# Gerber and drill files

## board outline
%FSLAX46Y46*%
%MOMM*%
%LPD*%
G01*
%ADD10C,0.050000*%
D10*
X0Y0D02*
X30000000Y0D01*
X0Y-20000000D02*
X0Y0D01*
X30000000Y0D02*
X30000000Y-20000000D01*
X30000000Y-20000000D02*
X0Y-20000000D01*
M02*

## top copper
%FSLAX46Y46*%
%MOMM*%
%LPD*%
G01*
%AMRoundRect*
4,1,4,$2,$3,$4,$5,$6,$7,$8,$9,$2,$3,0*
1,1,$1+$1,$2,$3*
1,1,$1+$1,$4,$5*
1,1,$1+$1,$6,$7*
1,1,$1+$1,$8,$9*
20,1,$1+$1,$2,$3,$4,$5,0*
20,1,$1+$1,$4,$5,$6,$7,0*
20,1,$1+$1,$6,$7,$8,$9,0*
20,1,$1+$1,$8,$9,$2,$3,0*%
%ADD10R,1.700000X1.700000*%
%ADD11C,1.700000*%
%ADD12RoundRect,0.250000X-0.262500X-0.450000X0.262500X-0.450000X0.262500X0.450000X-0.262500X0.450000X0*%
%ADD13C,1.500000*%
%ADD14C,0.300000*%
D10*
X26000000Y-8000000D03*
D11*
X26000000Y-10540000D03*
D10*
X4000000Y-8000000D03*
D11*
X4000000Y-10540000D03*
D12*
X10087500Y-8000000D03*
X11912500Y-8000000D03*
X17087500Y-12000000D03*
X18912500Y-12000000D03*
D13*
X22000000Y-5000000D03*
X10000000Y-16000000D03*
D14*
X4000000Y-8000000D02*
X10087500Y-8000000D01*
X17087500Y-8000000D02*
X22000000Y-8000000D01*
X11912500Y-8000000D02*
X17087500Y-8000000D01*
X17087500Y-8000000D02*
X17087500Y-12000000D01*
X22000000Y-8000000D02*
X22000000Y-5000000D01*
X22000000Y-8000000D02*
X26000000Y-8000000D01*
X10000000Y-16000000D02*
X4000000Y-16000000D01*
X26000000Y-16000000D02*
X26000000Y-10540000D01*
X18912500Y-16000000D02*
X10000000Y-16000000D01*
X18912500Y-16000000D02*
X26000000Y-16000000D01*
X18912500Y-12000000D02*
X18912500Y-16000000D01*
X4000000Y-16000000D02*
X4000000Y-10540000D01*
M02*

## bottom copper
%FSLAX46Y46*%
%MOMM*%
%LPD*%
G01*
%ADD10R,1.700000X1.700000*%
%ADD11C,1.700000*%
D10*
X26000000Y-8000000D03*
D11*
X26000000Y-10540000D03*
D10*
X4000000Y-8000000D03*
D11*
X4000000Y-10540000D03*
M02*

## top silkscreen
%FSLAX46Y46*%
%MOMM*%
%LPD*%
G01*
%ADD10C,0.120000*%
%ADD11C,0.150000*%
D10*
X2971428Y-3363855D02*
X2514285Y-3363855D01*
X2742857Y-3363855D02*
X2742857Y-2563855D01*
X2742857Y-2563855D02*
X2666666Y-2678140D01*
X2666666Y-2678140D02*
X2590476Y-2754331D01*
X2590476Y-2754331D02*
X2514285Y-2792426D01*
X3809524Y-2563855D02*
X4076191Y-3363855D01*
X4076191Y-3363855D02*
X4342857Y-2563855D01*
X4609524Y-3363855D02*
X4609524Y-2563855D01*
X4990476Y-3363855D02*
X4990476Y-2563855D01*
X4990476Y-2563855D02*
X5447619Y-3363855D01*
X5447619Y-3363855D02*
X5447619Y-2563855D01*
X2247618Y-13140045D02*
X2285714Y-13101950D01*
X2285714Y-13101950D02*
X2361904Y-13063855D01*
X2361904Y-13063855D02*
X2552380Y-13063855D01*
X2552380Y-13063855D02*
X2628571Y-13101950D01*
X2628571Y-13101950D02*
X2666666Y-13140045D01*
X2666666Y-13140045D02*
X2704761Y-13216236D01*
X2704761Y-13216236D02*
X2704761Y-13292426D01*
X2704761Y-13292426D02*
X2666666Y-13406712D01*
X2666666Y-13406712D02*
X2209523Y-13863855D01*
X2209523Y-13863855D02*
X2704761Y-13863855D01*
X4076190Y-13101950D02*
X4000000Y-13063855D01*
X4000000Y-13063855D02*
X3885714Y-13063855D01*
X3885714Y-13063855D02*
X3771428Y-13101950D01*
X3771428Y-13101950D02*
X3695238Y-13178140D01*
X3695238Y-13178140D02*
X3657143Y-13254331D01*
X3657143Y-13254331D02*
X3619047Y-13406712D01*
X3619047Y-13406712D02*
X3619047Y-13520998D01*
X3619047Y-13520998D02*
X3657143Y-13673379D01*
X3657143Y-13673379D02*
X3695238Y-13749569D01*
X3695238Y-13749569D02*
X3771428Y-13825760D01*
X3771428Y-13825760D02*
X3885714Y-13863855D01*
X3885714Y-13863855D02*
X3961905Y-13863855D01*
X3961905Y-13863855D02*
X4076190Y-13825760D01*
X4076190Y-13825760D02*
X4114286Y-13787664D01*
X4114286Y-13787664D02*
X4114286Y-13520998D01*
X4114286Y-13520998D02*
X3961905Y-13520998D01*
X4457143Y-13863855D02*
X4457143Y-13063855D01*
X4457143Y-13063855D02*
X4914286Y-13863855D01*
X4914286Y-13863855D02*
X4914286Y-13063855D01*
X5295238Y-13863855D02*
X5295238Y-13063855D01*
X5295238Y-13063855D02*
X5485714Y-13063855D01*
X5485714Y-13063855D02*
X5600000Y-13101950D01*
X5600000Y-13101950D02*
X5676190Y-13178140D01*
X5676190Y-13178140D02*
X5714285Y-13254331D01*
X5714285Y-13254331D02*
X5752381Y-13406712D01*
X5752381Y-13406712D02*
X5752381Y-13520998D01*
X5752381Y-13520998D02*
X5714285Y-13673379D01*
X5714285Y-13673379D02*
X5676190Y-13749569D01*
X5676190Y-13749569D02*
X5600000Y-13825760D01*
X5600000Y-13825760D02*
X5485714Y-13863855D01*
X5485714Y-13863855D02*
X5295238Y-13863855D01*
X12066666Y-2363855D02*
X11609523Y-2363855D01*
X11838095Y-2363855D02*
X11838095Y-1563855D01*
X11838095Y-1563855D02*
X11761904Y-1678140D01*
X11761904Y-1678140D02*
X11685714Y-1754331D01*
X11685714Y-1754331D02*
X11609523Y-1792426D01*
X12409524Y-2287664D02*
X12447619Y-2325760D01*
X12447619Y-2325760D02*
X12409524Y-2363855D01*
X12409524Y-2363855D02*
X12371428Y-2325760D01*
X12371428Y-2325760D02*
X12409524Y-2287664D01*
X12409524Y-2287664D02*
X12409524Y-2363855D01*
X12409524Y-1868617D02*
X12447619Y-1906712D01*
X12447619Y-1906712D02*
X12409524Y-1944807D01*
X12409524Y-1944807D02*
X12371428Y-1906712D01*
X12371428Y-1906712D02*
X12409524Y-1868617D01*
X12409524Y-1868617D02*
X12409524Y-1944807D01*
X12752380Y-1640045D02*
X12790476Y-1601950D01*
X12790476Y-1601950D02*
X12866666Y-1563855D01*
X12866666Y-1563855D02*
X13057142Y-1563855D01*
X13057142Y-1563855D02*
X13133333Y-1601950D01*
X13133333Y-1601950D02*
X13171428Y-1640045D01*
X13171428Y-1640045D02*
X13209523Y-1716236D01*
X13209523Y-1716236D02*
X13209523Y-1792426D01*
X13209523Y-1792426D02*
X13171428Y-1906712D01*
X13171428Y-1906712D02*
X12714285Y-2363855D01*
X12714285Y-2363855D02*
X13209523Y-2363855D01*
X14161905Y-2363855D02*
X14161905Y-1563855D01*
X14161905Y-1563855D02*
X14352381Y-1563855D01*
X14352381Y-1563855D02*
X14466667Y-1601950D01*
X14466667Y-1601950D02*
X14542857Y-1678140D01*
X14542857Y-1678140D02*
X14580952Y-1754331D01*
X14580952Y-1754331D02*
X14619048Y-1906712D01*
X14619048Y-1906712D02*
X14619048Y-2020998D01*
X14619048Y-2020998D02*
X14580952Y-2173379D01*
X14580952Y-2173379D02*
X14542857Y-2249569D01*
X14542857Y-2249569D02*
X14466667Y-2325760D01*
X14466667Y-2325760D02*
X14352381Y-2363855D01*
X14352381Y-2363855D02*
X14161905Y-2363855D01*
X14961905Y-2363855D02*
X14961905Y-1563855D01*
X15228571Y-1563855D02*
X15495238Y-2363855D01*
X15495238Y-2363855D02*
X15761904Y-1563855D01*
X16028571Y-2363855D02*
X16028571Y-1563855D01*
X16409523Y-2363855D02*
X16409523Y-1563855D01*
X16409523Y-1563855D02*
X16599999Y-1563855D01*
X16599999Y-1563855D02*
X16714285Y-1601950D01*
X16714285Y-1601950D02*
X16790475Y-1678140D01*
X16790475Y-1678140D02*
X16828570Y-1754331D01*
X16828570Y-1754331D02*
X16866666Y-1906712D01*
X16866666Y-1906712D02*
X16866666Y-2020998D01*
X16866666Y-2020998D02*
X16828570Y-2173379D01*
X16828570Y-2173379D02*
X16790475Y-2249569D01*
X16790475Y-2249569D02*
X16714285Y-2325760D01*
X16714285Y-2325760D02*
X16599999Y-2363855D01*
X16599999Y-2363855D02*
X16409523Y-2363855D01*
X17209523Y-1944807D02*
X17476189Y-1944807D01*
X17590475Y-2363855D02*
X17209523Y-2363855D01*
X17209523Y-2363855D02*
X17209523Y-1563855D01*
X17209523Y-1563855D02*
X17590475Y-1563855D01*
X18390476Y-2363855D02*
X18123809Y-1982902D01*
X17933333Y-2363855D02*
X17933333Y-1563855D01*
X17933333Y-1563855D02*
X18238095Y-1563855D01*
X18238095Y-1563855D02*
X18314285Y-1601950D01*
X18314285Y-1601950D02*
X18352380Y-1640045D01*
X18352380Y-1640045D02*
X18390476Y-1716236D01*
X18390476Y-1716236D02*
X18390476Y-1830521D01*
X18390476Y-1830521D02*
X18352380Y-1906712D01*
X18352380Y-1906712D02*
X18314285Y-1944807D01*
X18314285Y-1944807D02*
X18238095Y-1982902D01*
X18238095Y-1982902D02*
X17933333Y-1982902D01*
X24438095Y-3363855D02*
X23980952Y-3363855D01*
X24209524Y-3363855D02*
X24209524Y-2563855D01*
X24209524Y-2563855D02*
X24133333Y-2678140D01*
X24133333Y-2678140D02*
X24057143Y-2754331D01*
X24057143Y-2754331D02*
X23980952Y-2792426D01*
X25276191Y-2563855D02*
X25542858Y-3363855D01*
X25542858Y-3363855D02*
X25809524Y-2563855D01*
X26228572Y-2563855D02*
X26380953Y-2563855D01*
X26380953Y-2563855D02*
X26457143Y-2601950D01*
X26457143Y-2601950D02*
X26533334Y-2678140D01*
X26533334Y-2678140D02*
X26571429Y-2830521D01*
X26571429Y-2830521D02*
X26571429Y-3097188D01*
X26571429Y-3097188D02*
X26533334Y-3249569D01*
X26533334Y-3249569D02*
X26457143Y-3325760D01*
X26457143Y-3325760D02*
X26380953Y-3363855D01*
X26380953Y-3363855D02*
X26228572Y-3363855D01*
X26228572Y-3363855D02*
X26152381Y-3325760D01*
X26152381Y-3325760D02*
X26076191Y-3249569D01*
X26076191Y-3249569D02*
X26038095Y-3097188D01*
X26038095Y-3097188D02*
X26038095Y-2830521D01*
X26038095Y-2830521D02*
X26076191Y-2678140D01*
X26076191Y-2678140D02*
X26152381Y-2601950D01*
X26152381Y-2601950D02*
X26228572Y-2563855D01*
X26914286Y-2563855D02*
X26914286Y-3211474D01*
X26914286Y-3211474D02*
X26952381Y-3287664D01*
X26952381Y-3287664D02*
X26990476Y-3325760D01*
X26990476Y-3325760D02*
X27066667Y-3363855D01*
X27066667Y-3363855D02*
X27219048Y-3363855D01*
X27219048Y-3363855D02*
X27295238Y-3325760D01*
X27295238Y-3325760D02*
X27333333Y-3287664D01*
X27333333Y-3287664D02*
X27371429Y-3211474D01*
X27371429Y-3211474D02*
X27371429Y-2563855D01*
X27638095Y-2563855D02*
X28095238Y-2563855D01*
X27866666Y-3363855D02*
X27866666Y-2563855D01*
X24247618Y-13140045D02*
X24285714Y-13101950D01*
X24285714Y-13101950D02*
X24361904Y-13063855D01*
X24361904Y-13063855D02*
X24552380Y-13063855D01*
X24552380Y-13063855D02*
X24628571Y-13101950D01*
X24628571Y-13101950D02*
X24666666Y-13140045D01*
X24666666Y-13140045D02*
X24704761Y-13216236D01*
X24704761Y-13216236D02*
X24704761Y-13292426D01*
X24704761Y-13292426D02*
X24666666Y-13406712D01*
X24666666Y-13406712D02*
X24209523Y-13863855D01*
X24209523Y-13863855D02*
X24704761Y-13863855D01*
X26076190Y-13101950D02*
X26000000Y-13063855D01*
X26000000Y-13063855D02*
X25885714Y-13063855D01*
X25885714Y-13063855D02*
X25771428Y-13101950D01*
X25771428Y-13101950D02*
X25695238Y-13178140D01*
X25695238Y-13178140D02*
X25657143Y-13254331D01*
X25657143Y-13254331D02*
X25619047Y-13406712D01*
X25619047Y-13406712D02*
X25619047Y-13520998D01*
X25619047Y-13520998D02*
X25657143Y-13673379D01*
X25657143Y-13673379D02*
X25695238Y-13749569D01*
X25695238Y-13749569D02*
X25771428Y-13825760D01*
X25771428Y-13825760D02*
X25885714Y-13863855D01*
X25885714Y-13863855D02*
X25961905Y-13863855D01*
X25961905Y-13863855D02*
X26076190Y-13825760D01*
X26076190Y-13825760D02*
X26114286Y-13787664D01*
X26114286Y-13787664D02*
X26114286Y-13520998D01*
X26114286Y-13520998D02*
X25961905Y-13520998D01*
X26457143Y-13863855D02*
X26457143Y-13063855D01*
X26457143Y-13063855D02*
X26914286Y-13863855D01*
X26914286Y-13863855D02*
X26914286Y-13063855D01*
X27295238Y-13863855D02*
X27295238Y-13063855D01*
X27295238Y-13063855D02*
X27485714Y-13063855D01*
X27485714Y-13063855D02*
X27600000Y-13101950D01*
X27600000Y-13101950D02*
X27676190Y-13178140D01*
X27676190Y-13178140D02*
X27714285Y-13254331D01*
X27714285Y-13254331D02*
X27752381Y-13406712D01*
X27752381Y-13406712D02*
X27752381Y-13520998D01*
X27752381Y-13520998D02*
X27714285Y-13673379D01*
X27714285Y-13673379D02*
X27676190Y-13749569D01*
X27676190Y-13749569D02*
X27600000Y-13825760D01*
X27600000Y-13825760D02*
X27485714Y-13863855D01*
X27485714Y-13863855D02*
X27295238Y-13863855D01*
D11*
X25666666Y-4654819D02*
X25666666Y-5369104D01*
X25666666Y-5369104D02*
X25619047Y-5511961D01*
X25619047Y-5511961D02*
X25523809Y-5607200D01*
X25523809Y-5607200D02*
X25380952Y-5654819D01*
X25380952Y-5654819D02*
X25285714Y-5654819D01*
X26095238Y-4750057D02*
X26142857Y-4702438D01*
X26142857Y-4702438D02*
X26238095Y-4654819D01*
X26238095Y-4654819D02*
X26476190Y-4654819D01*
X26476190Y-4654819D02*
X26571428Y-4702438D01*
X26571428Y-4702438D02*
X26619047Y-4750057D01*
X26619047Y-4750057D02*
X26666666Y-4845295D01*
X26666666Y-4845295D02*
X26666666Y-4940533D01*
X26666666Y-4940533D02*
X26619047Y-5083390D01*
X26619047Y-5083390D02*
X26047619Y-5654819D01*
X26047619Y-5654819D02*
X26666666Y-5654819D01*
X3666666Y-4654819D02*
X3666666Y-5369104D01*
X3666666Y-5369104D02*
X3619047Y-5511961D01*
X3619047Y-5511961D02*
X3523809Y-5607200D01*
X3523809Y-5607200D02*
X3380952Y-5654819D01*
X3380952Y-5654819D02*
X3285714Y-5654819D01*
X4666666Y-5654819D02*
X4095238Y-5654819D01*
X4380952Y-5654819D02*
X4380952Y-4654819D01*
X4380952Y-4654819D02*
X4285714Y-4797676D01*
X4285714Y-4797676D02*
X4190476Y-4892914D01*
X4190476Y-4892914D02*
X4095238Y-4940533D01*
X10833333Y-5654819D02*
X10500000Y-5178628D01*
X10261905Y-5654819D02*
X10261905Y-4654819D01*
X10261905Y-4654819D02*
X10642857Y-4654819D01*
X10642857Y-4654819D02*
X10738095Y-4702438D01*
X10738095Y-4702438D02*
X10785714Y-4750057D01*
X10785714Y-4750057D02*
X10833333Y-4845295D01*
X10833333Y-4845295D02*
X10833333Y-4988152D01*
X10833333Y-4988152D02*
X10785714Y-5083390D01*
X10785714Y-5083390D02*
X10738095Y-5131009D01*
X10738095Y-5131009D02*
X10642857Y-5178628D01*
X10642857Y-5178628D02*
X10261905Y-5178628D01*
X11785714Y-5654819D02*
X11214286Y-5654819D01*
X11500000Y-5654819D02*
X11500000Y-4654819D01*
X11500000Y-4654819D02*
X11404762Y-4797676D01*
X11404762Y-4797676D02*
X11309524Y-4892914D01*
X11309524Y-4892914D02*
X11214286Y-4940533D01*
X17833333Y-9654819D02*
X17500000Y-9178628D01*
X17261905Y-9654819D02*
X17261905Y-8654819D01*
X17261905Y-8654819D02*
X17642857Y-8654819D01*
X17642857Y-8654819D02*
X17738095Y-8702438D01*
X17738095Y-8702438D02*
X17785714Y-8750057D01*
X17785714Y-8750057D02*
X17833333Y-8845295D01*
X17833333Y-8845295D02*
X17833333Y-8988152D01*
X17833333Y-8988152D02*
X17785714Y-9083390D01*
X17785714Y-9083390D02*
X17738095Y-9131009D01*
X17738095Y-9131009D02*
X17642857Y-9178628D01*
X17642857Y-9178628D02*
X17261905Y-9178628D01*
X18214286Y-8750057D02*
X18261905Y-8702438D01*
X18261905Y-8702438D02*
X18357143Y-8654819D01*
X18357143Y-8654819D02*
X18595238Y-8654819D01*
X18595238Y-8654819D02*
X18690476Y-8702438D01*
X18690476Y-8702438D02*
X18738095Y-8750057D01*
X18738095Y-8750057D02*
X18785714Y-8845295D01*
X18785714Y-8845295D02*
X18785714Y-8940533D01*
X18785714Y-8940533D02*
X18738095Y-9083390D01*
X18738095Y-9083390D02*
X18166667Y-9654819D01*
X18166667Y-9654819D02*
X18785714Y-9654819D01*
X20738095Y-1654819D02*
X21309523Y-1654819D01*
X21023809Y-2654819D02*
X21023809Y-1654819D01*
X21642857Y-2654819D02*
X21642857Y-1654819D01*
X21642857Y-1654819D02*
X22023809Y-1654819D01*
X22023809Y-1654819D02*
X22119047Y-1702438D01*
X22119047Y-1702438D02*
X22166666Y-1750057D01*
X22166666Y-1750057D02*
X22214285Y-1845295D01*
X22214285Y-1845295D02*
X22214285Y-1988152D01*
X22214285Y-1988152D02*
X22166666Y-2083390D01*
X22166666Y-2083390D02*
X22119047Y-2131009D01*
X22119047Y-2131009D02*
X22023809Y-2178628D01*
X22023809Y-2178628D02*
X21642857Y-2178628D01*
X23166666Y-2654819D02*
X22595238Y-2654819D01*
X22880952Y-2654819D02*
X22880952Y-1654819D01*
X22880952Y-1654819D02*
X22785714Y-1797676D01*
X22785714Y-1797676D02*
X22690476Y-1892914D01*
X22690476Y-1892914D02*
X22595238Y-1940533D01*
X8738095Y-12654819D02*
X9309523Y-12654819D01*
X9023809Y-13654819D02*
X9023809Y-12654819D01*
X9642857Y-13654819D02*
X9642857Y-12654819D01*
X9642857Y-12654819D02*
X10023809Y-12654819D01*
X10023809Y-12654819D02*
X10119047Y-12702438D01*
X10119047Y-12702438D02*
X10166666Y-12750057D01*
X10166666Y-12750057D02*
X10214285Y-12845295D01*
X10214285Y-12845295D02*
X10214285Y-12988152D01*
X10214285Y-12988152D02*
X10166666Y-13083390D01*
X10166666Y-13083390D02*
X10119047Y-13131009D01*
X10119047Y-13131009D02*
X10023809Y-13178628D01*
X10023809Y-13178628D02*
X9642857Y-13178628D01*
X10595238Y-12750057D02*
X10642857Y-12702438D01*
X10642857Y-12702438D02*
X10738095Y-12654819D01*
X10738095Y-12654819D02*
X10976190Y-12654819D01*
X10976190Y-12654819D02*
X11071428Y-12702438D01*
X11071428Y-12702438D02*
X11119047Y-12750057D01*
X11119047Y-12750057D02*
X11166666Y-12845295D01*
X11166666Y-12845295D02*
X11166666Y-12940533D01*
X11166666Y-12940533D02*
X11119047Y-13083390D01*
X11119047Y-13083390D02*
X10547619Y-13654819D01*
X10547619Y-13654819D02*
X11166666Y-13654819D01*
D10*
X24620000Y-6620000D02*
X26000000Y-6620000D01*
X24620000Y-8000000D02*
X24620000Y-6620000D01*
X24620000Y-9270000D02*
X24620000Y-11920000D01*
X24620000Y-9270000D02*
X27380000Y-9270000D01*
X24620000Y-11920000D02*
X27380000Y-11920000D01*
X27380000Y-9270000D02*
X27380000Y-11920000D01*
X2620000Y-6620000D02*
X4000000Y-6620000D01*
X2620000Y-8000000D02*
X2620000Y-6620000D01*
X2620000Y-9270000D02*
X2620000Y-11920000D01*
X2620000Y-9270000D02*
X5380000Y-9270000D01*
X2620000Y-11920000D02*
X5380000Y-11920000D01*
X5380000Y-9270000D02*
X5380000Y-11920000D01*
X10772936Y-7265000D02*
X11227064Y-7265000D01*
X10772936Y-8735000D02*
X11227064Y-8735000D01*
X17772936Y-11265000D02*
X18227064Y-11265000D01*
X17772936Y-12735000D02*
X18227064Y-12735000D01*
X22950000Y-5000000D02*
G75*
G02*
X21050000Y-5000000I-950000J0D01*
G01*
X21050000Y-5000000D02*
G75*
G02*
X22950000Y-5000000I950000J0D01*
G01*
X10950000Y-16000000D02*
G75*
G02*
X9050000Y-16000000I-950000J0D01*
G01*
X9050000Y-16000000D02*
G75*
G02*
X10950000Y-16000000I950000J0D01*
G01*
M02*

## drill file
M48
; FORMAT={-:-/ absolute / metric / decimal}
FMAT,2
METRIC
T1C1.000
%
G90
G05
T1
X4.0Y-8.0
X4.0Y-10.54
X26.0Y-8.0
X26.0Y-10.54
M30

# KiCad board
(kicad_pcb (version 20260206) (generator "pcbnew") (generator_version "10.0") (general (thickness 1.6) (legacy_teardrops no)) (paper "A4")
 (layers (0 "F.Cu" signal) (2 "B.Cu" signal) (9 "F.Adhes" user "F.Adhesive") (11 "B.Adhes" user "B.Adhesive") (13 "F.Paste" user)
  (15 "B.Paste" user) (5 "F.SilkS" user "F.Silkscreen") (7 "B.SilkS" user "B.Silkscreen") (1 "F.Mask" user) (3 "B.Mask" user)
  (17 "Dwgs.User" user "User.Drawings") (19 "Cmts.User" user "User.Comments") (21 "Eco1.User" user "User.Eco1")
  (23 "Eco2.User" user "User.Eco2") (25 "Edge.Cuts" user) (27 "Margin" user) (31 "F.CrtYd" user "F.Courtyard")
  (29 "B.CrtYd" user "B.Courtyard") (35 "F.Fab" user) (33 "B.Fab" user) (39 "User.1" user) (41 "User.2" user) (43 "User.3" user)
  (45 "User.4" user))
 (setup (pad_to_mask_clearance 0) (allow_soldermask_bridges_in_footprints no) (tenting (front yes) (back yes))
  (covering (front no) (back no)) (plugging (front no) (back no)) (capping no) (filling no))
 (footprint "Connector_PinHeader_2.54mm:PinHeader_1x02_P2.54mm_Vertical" (layer "F.Cu") (at 26 8)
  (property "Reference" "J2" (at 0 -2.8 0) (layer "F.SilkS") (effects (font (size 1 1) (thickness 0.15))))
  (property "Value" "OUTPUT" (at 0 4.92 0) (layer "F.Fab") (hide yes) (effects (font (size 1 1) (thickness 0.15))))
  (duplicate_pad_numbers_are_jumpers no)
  (fp_line (start -1.38 -1.38) (end 0 -1.38) (stroke (width 0.12) (type solid)) (layer "F.SilkS"))
  (fp_line (start -1.38 0) (end -1.38 -1.38) (stroke (width 0.12) (type solid)) (layer "F.SilkS"))
  (fp_line (start -1.38 1.27) (end -1.38 3.92) (stroke (width 0.12) (type solid)) (layer "F.SilkS"))
  (fp_line (start -1.38 1.27) (end 1.38 1.27) (stroke (width 0.12) (type solid)) (layer "F.SilkS"))
  (fp_line (start -1.38 3.92) (end 1.38 3.92) (stroke (width 0.12) (type solid)) (layer "F.SilkS"))
  (fp_line (start 1.38 1.27) (end 1.38 3.92) (stroke (width 0.12) (type solid)) (layer "F.SilkS"))
  (pad "1" thru_hole rect (at 0 0) (size 1.7 1.7) (drill 1) (layers "*.Cu" "*.Mask") (remove_unused_layers no) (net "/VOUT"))
  (pad "2" thru_hole circle (at 0 2.54) (size 1.7 1.7) (drill 1) (layers "*.Cu" "*.Mask") (remove_unused_layers no) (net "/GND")))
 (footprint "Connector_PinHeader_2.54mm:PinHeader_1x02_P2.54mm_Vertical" (layer "F.Cu") (at 4 8)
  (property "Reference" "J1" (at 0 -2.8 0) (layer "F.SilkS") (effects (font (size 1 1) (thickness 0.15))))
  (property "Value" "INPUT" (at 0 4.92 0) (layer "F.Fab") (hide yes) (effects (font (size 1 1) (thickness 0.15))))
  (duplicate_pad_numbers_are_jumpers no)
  (fp_line (start -1.38 -1.38) (end 0 -1.38) (stroke (width 0.12) (type solid)) (layer "F.SilkS"))
  (fp_line (start -1.38 0) (end -1.38 -1.38) (stroke (width 0.12) (type solid)) (layer "F.SilkS"))
  (fp_line (start -1.38 1.27) (end -1.38 3.92) (stroke (width 0.12) (type solid)) (layer "F.SilkS"))
  (fp_line (start -1.38 1.27) (end 1.38 1.27) (stroke (width 0.12) (type solid)) (layer "F.SilkS"))
  (fp_line (start -1.38 3.92) (end 1.38 3.92) (stroke (width 0.12) (type solid)) (layer "F.SilkS"))
  (fp_line (start 1.38 1.27) (end 1.38 3.92) (stroke (width 0.12) (type solid)) (layer "F.SilkS"))
  (pad "1" thru_hole rect (at 0 0) (size 1.7 1.7) (drill 1) (layers "*.Cu" "*.Mask") (remove_unused_layers no) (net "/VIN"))
  (pad "2" thru_hole circle (at 0 2.54) (size 1.7 1.7) (drill 1) (layers "*.Cu" "*.Mask") (remove_unused_layers no) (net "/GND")))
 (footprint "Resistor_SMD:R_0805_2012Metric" (layer "F.Cu") (at 11 8)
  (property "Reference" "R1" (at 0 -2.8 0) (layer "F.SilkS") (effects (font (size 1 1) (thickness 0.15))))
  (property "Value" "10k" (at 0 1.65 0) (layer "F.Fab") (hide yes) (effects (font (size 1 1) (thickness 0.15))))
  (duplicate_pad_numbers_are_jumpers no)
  (fp_line (start -0.227064 -0.735) (end 0.227064 -0.735) (stroke (width 0.12) (type solid)) (layer "F.SilkS"))
  (fp_line (start -0.227064 0.735) (end 0.227064 0.735) (stroke (width 0.12) (type solid)) (layer "F.SilkS"))
  (pad "1" smd roundrect (at -0.9125 0) (size 1.025 1.4) (layers "F.Cu" "F.Mask" "F.Paste") (roundrect_rratio 0.243902) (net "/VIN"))
  (pad "2" smd roundrect (at 0.9125 0) (size 1.025 1.4) (layers "F.Cu" "F.Mask" "F.Paste") (roundrect_rratio 0.243902) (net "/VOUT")))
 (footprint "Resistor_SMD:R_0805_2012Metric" (layer "F.Cu") (at 18 12)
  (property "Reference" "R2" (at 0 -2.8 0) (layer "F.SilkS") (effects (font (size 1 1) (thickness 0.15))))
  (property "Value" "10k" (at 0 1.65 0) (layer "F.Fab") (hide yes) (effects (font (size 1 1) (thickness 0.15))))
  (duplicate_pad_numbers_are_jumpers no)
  (fp_line (start -0.227064 -0.735) (end 0.227064 -0.735) (stroke (width 0.12) (type solid)) (layer "F.SilkS"))
  (fp_line (start -0.227064 0.735) (end 0.227064 0.735) (stroke (width 0.12) (type solid)) (layer "F.SilkS"))
  (pad "1" smd roundrect (at -0.9125 0) (size 1.025 1.4) (layers "F.Cu" "F.Mask" "F.Paste") (roundrect_rratio 0.243902) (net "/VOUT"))
  (pad "2" smd roundrect (at 0.9125 0) (size 1.025 1.4) (layers "F.Cu" "F.Mask" "F.Paste") (roundrect_rratio 0.243902) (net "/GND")))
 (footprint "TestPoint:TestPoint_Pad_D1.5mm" (layer "F.Cu") (at 22 5)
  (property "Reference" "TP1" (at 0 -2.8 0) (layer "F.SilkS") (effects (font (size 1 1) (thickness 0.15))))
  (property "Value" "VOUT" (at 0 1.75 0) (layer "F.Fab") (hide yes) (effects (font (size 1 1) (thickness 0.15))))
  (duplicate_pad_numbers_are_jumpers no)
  (fp_circle (center 0 0) (end 0 0.95) (stroke (width 0.12) (type solid)) (fill no) (layer "F.SilkS"))
  (pad "1" smd circle (at 0 0) (size 1.5 1.5) (layers "F.Cu" "F.Mask") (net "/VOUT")))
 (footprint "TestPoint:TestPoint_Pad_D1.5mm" (layer "F.Cu") (at 10 16)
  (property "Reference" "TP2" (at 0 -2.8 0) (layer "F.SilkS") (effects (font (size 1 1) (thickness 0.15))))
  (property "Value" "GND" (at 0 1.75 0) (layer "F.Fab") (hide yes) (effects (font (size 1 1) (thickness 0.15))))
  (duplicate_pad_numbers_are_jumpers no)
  (fp_circle (center 0 0) (end 0 0.95) (stroke (width 0.12) (type solid)) (fill no) (layer "F.SilkS"))
  (pad "1" smd circle (at 0 0) (size 1.5 1.5) (layers "F.Cu" "F.Mask") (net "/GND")))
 (gr_line (start 0 0) (end 30 0) (stroke (width 0.05) (type default)) (layer "Edge.Cuts"))
 (gr_line (start 0 20) (end 0 0) (stroke (width 0.05) (type default)) (layer "Edge.Cuts"))
 (gr_line (start 30 0) (end 30 20) (stroke (width 0.05) (type default)) (layer "Edge.Cuts"))
 (gr_line (start 30 20) (end 0 20) (stroke (width 0.05) (type default)) (layer "Edge.Cuts"))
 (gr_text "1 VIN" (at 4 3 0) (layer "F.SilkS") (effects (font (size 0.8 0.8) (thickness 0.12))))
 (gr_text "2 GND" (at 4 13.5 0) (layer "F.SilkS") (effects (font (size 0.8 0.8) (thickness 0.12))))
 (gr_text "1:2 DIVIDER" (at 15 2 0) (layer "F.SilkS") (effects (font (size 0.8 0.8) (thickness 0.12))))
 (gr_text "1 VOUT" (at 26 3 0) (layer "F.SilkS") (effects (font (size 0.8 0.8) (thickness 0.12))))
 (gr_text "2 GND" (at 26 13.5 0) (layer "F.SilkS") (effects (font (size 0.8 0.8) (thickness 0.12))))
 (segment (start 4 8) (end 10.0875 8) (width 0.3) (layer "F.Cu") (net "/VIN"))
 (segment (start 17.0875 8) (end 22 8) (width 0.3) (layer "F.Cu") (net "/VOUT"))
 (segment (start 11.9125 8) (end 17.0875 8) (width 0.3) (layer "F.Cu") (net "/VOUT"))
 (segment (start 17.0875 8) (end 17.0875 12) (width 0.3) (layer "F.Cu") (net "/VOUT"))
 (segment (start 22 8) (end 22 5) (width 0.3) (layer "F.Cu") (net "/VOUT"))
 (segment (start 22 8) (end 26 8) (width 0.3) (layer "F.Cu") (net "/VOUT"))
 (segment (start 10 16) (end 4 16) (width 0.3) (layer "F.Cu") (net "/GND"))
 (segment (start 26 16) (end 26 10.54) (width 0.3) (layer "F.Cu") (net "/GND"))
 (segment (start 18.9125 16) (end 10 16) (width 0.3) (layer "F.Cu") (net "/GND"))
 (segment (start 18.9125 16) (end 26 16) (width 0.3) (layer "F.Cu") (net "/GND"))
 (segment (start 18.9125 12) (end 18.9125 16) (width 0.3) (layer "F.Cu") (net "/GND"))
 (segment (start 4 16) (end 4 10.54) (width 0.3) (layer "F.Cu") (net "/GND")))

